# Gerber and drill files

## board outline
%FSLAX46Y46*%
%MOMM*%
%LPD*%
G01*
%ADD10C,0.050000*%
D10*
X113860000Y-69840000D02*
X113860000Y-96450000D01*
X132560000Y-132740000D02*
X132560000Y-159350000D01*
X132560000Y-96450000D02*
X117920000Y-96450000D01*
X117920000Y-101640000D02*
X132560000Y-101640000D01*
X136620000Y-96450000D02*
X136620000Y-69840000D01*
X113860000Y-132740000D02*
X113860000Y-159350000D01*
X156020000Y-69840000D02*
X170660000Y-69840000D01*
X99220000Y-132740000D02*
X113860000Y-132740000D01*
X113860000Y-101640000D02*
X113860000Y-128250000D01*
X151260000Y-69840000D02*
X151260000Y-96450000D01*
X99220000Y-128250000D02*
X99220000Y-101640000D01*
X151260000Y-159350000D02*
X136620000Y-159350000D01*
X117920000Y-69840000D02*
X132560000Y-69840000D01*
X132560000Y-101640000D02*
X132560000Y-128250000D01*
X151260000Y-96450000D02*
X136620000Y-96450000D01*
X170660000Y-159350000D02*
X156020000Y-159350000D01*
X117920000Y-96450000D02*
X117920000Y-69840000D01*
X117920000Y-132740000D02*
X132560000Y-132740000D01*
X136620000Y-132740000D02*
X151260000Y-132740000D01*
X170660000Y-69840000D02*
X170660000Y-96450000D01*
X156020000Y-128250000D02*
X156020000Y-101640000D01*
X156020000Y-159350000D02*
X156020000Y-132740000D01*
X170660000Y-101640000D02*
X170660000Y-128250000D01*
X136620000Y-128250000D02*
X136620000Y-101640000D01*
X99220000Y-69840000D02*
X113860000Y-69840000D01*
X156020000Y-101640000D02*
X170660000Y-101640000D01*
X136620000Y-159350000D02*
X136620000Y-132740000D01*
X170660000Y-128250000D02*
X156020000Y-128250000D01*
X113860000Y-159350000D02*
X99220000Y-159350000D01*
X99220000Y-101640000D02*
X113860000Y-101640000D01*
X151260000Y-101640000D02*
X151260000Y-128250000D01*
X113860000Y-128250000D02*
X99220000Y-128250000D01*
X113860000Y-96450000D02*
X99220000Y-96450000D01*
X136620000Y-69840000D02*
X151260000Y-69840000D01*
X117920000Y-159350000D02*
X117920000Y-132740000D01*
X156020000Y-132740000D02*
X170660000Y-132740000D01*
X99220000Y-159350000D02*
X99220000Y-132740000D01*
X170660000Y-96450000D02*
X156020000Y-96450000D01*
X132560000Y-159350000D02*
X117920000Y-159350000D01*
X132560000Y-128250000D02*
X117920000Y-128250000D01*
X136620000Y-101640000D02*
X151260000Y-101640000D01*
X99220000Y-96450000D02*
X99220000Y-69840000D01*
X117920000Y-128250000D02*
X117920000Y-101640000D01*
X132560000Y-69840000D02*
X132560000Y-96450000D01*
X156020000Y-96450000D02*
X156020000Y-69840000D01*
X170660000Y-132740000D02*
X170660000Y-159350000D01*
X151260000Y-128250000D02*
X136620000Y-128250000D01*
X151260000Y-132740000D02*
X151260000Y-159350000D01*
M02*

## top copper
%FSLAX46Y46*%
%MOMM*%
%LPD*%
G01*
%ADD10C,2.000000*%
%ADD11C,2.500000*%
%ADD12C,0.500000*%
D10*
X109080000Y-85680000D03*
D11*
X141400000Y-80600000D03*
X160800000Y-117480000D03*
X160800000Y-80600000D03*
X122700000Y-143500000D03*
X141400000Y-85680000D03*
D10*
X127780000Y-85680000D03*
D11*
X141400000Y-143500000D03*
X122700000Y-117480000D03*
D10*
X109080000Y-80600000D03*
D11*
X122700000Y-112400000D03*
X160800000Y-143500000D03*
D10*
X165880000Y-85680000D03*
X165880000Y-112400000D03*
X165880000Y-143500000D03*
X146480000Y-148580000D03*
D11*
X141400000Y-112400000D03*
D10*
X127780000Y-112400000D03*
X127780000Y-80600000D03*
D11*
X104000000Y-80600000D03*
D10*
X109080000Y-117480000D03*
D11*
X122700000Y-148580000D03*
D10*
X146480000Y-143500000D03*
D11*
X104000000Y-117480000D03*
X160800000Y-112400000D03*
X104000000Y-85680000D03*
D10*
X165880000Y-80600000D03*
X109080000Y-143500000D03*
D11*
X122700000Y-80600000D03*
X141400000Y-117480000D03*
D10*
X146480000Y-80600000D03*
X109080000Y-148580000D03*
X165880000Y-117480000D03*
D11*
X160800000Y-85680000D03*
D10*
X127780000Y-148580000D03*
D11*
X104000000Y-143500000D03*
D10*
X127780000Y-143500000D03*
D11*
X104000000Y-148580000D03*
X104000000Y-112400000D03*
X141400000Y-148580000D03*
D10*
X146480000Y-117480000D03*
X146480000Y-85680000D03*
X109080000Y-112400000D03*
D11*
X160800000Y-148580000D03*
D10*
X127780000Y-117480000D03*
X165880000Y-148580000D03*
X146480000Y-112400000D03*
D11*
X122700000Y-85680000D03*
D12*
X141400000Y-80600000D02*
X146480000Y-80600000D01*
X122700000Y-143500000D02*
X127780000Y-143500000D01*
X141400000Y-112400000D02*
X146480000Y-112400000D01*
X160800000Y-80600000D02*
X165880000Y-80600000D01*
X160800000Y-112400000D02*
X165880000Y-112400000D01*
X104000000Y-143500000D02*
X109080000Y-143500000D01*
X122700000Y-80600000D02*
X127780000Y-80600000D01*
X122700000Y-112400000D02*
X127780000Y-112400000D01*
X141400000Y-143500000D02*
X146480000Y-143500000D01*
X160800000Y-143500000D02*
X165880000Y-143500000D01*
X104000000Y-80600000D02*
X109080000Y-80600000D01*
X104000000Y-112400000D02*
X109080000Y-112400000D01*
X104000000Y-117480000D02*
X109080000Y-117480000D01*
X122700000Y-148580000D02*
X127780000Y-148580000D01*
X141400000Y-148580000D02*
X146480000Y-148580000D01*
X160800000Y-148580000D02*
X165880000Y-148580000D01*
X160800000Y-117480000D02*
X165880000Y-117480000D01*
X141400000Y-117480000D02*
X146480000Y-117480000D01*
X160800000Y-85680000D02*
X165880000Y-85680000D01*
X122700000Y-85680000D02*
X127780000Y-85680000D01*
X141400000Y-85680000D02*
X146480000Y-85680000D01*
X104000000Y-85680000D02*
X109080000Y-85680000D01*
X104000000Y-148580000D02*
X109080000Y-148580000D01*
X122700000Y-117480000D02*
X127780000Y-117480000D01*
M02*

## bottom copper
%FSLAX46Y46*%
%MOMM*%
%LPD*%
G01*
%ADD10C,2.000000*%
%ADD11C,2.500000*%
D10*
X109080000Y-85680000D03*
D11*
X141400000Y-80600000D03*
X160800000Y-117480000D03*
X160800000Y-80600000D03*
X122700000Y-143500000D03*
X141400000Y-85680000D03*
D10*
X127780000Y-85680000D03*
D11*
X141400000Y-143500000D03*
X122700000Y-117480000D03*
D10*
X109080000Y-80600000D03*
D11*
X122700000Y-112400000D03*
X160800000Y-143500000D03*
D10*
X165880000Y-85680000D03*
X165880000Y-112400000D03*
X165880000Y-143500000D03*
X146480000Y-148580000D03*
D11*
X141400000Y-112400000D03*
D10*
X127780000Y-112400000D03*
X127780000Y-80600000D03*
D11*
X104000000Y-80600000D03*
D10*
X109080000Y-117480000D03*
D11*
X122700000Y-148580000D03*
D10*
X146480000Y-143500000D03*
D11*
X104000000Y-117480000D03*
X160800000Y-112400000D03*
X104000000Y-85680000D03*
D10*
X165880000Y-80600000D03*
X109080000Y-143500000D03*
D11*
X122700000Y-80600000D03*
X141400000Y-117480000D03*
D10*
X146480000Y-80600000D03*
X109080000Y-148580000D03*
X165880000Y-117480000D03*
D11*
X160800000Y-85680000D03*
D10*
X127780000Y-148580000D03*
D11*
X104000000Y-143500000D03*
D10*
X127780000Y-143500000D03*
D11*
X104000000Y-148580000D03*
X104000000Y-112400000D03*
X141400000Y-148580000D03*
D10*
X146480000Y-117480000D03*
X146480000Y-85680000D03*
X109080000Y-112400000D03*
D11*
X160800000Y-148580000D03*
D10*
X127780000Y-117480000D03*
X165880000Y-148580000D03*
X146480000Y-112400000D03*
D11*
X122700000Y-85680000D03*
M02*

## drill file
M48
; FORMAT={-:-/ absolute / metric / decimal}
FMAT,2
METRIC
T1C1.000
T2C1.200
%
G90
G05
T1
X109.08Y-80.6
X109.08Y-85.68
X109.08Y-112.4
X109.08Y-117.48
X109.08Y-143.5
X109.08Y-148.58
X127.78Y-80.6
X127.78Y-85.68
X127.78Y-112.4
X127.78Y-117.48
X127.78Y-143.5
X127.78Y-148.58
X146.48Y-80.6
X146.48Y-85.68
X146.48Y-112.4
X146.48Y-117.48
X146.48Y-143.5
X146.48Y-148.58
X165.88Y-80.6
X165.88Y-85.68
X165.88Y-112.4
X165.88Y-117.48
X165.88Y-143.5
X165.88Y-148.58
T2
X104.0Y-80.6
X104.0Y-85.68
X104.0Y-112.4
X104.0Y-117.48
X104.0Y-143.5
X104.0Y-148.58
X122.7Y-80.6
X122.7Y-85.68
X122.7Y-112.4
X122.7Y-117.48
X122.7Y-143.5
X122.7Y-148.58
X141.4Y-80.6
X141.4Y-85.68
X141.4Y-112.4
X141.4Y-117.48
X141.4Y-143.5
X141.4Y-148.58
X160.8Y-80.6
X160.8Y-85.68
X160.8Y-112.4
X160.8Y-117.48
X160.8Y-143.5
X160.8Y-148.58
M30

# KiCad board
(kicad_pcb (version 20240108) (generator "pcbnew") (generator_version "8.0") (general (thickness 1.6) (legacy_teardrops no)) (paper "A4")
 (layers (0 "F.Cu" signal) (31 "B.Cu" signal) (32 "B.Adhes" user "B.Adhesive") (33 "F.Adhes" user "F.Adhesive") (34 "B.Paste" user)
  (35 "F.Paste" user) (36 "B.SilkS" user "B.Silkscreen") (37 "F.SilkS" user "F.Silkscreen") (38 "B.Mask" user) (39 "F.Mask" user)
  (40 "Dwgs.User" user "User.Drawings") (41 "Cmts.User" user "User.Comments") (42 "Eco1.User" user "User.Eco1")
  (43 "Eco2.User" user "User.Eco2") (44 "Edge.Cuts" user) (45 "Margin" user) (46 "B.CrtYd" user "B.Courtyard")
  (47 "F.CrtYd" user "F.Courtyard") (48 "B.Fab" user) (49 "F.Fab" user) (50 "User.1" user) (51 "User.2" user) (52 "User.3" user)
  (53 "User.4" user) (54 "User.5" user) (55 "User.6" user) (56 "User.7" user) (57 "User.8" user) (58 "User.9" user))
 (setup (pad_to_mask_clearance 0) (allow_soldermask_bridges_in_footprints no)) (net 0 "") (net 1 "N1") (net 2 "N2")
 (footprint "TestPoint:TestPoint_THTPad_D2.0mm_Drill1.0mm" (layer "F.Cu") (at 109.08 85.68)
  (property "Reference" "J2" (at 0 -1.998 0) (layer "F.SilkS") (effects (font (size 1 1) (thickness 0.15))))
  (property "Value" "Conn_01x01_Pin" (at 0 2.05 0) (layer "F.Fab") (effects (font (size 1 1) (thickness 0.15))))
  (pad "1" thru_hole circle (at 0 0) (size 2 2) (drill 1) (layers "*.Cu" "*.Mask") (remove_unused_layers no) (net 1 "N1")))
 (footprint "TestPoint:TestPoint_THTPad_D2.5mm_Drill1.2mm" (layer "F.Cu") (at 141.4 80.6)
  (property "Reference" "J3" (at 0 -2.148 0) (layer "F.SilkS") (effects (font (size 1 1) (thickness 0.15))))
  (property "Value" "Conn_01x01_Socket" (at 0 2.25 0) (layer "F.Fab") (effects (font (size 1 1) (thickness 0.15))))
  (pad "1" thru_hole circle (at 0 0) (size 2.5 2.5) (drill 1.2) (layers "*.Cu" "*.Mask") (remove_unused_layers no) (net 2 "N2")))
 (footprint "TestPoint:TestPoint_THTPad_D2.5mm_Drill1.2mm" (layer "F.Cu") (at 160.8 117.48)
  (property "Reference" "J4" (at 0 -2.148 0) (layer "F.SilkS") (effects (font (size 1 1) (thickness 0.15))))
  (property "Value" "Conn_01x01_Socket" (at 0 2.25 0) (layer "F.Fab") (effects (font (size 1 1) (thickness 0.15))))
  (pad "1" thru_hole circle (at 0 0) (size 2.5 2.5) (drill 1.2) (layers "*.Cu" "*.Mask") (remove_unused_layers no) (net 1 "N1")))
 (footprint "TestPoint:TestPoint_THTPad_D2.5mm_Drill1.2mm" (layer "F.Cu") (at 160.8 80.6)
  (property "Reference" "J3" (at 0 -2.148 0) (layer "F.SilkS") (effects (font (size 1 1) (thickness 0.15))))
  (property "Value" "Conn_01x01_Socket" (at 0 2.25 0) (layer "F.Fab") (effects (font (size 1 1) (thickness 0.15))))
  (pad "1" thru_hole circle (at 0 0) (size 2.5 2.5) (drill 1.2) (layers "*.Cu" "*.Mask") (remove_unused_layers no) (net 2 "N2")))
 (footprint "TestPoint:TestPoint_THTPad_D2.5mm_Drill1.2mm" (layer "F.Cu") (at 122.7 143.5)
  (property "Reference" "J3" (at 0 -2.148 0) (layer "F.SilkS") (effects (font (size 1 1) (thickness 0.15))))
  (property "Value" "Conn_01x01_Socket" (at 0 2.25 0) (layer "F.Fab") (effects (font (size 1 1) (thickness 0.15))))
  (pad "1" thru_hole circle (at 0 0) (size 2.5 2.5) (drill 1.2) (layers "*.Cu" "*.Mask") (remove_unused_layers no) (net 2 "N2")))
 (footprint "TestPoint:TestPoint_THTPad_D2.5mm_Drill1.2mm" (layer "F.Cu") (at 141.4 85.68)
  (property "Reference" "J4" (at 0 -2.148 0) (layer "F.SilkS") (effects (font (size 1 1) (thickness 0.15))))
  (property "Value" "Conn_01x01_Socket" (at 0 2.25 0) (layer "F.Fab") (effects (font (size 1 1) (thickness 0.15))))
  (pad "1" thru_hole circle (at 0 0) (size 2.5 2.5) (drill 1.2) (layers "*.Cu" "*.Mask") (remove_unused_layers no) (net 1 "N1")))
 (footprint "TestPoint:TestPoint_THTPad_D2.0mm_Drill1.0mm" (layer "F.Cu") (at 127.78 85.68)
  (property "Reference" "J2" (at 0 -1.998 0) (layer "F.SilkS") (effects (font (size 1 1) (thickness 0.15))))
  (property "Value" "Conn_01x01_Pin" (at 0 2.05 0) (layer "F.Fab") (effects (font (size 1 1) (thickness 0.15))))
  (pad "1" thru_hole circle (at 0 0) (size 2 2) (drill 1) (layers "*.Cu" "*.Mask") (remove_unused_layers no) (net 1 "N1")))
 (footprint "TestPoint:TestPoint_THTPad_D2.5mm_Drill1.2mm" (layer "F.Cu") (at 141.4 143.5)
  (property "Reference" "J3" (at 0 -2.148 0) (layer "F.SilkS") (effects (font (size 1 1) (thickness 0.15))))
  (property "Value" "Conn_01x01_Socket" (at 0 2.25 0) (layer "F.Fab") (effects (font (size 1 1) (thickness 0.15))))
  (pad "1" thru_hole circle (at 0 0) (size 2.5 2.5) (drill 1.2) (layers "*.Cu" "*.Mask") (remove_unused_layers no) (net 2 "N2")))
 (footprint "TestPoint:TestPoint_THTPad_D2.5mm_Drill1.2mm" (layer "F.Cu") (at 122.7 117.48)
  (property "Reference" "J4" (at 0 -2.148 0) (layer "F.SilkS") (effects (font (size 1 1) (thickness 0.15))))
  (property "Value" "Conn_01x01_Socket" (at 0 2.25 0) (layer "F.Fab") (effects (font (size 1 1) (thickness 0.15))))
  (pad "1" thru_hole circle (at 0 0) (size 2.5 2.5) (drill 1.2) (layers "*.Cu" "*.Mask") (remove_unused_layers no) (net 1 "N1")))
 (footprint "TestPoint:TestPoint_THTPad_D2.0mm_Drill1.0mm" (layer "F.Cu") (at 109.08 80.6)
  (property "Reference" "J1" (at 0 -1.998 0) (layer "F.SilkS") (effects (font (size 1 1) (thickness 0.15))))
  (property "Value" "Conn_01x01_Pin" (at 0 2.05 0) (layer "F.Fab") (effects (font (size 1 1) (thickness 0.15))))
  (pad "1" thru_hole circle (at 0 0) (size 2 2) (drill 1) (layers "*.Cu" "*.Mask") (remove_unused_layers no) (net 2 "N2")))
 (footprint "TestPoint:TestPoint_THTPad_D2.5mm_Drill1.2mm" (layer "F.Cu") (at 122.7 112.4)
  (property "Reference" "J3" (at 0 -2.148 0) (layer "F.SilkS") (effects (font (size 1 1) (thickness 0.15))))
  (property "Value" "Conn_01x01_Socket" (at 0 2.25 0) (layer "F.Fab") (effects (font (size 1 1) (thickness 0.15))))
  (pad "1" thru_hole circle (at 0 0) (size 2.5 2.5) (drill 1.2) (layers "*.Cu" "*.Mask") (remove_unused_layers no) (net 2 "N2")))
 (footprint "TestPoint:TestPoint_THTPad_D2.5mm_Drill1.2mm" (layer "F.Cu") (at 160.8 143.5)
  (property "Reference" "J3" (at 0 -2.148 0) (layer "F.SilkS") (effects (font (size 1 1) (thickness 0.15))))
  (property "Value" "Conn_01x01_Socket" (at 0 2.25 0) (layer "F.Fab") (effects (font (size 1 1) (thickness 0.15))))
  (pad "1" thru_hole circle (at 0 0) (size 2.5 2.5) (drill 1.2) (layers "*.Cu" "*.Mask") (remove_unused_layers no) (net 2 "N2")))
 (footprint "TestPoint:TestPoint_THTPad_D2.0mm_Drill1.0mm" (layer "F.Cu") (at 165.88 85.68)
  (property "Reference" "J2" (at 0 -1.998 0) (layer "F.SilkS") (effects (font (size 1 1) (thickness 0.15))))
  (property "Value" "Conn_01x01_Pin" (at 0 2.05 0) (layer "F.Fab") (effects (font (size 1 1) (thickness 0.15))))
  (pad "1" thru_hole circle (at 0 0) (size 2 2) (drill 1) (layers "*.Cu" "*.Mask") (remove_unused_layers no) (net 1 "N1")))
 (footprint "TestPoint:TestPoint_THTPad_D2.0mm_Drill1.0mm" (layer "F.Cu") (at 165.88 112.4)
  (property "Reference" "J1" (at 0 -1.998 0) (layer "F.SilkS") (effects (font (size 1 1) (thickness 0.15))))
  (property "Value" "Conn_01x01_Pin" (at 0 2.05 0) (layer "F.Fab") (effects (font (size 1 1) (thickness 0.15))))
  (pad "1" thru_hole circle (at 0 0) (size 2 2) (drill 1) (layers "*.Cu" "*.Mask") (remove_unused_layers no) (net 2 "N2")))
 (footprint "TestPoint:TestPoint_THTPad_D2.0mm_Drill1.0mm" (layer "F.Cu") (at 165.88 143.5)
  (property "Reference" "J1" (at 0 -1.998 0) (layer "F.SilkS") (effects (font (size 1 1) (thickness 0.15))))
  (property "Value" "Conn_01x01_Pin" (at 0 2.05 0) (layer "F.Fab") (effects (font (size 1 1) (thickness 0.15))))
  (pad "1" thru_hole circle (at 0 0) (size 2 2) (drill 1) (layers "*.Cu" "*.Mask") (remove_unused_layers no) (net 2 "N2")))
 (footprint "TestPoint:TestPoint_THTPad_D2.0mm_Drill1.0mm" (layer "F.Cu") (at 146.48 148.58)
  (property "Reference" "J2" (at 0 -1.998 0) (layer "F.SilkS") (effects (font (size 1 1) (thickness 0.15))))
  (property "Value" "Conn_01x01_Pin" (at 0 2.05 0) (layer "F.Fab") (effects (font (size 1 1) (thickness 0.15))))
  (pad "1" thru_hole circle (at 0 0) (size 2 2) (drill 1) (layers "*.Cu" "*.Mask") (remove_unused_layers no) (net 1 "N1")))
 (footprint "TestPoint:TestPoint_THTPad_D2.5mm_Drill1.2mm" (layer "F.Cu") (at 141.4 112.4)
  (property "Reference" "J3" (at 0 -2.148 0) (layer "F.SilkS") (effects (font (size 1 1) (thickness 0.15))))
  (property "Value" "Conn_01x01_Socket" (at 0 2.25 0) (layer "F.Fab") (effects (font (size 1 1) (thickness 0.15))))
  (pad "1" thru_hole circle (at 0 0) (size 2.5 2.5) (drill 1.2) (layers "*.Cu" "*.Mask") (remove_unused_layers no) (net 2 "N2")))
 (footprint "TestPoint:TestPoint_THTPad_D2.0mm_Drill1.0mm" (layer "F.Cu") (at 127.78 112.4)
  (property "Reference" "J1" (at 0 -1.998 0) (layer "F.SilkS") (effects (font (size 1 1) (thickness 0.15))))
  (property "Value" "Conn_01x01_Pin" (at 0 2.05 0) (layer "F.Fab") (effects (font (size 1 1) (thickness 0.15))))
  (pad "1" thru_hole circle (at 0 0) (size 2 2) (drill 1) (layers "*.Cu" "*.Mask") (remove_unused_layers no) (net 2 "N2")))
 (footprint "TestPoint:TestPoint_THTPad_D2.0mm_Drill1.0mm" (layer "F.Cu") (at 127.78 80.6)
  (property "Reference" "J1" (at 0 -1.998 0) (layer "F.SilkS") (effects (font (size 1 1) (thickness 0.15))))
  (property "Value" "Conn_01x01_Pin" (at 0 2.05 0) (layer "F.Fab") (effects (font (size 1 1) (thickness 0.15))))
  (pad "1" thru_hole circle (at 0 0) (size 2 2) (drill 1) (layers "*.Cu" "*.Mask") (remove_unused_layers no) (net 2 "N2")))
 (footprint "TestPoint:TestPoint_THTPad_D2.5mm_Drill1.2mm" (layer "F.Cu") (at 104 80.6)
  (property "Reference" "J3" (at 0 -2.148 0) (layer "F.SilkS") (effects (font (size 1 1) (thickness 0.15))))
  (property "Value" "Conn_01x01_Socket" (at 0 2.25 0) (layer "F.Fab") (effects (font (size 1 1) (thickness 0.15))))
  (pad "1" thru_hole circle (at 0 0) (size 2.5 2.5) (drill 1.2) (layers "*.Cu" "*.Mask") (remove_unused_layers no) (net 2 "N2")))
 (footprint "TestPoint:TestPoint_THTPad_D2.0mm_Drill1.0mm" (layer "F.Cu") (at 109.08 117.48)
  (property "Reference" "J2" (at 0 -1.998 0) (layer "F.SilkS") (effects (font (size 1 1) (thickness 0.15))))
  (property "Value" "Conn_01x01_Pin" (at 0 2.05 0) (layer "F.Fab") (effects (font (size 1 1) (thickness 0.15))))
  (pad "1" thru_hole circle (at 0 0) (size 2 2) (drill 1) (layers "*.Cu" "*.Mask") (remove_unused_layers no) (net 1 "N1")))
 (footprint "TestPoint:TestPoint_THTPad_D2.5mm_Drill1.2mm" (layer "F.Cu") (at 122.7 148.58)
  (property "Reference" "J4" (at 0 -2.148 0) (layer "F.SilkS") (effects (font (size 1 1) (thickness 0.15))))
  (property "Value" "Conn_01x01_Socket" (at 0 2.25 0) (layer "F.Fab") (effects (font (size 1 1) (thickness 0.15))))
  (pad "1" thru_hole circle (at 0 0) (size 2.5 2.5) (drill 1.2) (layers "*.Cu" "*.Mask") (remove_unused_layers no) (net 1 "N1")))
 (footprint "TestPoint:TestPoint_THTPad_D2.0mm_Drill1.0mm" (layer "F.Cu") (at 146.48 143.5)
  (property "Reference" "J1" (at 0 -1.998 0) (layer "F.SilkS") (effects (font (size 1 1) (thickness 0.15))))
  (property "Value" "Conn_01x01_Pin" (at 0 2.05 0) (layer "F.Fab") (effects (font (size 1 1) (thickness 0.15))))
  (pad "1" thru_hole circle (at 0 0) (size 2 2) (drill 1) (layers "*.Cu" "*.Mask") (remove_unused_layers no) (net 2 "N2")))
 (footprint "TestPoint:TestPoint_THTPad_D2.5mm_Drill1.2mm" (layer "F.Cu") (at 104 117.48)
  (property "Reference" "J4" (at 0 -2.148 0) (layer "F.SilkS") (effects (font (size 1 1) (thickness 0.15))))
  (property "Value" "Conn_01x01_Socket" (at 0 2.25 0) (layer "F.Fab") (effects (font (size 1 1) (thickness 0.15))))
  (pad "1" thru_hole circle (at 0 0) (size 2.5 2.5) (drill 1.2) (layers "*.Cu" "*.Mask") (remove_unused_layers no) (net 1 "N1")))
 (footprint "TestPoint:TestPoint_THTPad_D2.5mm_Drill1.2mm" (layer "F.Cu") (at 160.8 112.4)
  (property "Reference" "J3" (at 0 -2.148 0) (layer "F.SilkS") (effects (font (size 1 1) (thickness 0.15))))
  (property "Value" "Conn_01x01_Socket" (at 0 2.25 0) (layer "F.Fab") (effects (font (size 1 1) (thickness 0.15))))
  (pad "1" thru_hole circle (at 0 0) (size 2.5 2.5) (drill 1.2) (layers "*.Cu" "*.Mask") (remove_unused_layers no) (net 2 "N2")))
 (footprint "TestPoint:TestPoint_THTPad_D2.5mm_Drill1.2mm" (layer "F.Cu") (at 104 85.68)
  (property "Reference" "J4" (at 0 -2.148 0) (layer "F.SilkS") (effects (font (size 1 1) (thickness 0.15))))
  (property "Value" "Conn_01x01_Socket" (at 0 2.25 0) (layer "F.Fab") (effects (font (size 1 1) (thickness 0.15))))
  (pad "1" thru_hole circle (at 0 0) (size 2.5 2.5) (drill 1.2) (layers "*.Cu" "*.Mask") (remove_unused_layers no) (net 1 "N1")))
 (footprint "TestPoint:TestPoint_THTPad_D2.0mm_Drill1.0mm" (layer "F.Cu") (at 165.88 80.6)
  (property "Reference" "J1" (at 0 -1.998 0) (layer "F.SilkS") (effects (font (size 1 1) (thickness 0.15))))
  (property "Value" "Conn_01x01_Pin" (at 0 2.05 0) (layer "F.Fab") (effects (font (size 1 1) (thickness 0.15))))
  (pad "1" thru_hole circle (at 0 0) (size 2 2) (drill 1) (layers "*.Cu" "*.Mask") (remove_unused_layers no) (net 2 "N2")))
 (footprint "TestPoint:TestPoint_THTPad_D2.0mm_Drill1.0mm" (layer "F.Cu") (at 109.08 143.5)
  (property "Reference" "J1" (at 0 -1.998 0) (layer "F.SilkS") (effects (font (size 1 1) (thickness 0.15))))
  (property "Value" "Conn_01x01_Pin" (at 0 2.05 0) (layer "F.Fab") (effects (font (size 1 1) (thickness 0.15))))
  (pad "1" thru_hole circle (at 0 0) (size 2 2) (drill 1) (layers "*.Cu" "*.Mask") (remove_unused_layers no) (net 2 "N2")))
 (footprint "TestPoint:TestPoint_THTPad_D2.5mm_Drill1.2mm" (layer "F.Cu") (at 122.7 80.6)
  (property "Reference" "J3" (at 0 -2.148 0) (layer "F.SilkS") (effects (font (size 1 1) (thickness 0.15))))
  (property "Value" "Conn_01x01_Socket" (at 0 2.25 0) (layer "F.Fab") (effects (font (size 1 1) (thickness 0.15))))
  (pad "1" thru_hole circle (at 0 0) (size 2.5 2.5) (drill 1.2) (layers "*.Cu" "*.Mask") (remove_unused_layers no) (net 2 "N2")))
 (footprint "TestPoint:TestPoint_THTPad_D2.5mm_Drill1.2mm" (layer "F.Cu") (at 141.4 117.48)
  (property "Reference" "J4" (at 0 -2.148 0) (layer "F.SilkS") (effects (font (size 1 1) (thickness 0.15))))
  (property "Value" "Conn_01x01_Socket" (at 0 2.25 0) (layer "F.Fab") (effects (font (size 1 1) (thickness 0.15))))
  (pad "1" thru_hole circle (at 0 0) (size 2.5 2.5) (drill 1.2) (layers "*.Cu" "*.Mask") (remove_unused_layers no) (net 1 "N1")))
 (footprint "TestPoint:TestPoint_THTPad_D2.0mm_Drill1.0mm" (layer "F.Cu") (at 146.48 80.6)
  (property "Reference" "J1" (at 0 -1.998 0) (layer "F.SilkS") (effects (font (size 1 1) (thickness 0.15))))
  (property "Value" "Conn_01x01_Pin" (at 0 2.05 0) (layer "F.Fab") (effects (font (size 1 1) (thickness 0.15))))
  (pad "1" thru_hole circle (at 0 0) (size 2 2) (drill 1) (layers "*.Cu" "*.Mask") (remove_unused_layers no) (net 2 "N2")))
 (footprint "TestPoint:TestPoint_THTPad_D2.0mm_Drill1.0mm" (layer "F.Cu") (at 109.08 148.58)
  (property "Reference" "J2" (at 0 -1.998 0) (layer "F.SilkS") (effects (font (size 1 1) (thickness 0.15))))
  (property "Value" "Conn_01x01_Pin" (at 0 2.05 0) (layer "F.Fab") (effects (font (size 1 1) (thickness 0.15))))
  (pad "1" thru_hole circle (at 0 0) (size 2 2) (drill 1) (layers "*.Cu" "*.Mask") (remove_unused_layers no) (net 1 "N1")))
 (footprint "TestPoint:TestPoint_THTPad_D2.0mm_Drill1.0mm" (layer "F.Cu") (at 165.88 117.48)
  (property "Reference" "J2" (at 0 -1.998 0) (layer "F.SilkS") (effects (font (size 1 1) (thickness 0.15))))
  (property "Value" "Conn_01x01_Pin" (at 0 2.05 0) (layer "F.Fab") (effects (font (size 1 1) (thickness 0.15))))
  (pad "1" thru_hole circle (at 0 0) (size 2 2) (drill 1) (layers "*.Cu" "*.Mask") (remove_unused_layers no) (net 1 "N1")))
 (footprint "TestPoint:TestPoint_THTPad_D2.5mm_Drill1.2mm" (layer "F.Cu") (at 160.8 85.68)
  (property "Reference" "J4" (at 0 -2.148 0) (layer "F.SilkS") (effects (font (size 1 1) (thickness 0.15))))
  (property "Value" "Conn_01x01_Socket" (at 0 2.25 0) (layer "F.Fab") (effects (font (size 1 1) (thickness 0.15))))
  (pad "1" thru_hole circle (at 0 0) (size 2.5 2.5) (drill 1.2) (layers "*.Cu" "*.Mask") (remove_unused_layers no) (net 1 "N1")))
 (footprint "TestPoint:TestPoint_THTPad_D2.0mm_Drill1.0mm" (layer "F.Cu") (at 127.78 148.58)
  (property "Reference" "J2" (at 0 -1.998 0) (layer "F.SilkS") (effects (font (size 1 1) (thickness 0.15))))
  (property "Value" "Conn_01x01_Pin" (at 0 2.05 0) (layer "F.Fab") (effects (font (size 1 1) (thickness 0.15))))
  (pad "1" thru_hole circle (at 0 0) (size 2 2) (drill 1) (layers "*.Cu" "*.Mask") (remove_unused_layers no) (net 1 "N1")))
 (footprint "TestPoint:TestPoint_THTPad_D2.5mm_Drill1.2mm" (layer "F.Cu") (at 104 143.5)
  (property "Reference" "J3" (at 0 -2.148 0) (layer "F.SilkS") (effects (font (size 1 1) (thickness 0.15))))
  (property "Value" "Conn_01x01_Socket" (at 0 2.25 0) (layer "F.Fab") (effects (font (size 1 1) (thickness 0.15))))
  (pad "1" thru_hole circle (at 0 0) (size 2.5 2.5) (drill 1.2) (layers "*.Cu" "*.Mask") (remove_unused_layers no) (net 2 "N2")))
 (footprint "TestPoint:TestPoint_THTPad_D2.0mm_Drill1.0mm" (layer "F.Cu") (at 127.78 143.5)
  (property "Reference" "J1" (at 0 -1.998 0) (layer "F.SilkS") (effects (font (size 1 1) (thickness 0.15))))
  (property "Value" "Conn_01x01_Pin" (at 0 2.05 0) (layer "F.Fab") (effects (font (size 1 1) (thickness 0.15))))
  (pad "1" thru_hole circle (at 0 0) (size 2 2) (drill 1) (layers "*.Cu" "*.Mask") (remove_unused_layers no) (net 2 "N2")))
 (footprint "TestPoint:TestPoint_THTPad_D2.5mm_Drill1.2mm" (layer "F.Cu") (at 104 148.58)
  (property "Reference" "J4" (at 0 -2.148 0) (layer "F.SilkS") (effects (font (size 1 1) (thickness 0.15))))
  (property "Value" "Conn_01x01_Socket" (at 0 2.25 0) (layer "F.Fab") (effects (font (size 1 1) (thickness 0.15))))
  (pad "1" thru_hole circle (at 0 0) (size 2.5 2.5) (drill 1.2) (layers "*.Cu" "*.Mask") (remove_unused_layers no) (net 1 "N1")))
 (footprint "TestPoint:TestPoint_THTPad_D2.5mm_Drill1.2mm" (layer "F.Cu") (at 104 112.4)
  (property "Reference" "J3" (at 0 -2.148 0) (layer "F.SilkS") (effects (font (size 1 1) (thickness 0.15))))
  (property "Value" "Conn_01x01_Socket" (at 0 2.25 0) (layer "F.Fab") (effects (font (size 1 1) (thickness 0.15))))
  (pad "1" thru_hole circle (at 0 0) (size 2.5 2.5) (drill 1.2) (layers "*.Cu" "*.Mask") (remove_unused_layers no) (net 2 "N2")))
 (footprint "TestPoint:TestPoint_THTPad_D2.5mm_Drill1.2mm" (layer "F.Cu") (at 141.4 148.58)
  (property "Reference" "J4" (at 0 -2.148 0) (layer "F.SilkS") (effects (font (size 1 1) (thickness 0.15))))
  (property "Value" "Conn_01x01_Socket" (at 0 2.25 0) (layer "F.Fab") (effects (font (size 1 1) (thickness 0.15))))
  (pad "1" thru_hole circle (at 0 0) (size 2.5 2.5) (drill 1.2) (layers "*.Cu" "*.Mask") (remove_unused_layers no) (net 1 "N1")))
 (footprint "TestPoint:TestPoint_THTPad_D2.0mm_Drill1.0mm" (layer "F.Cu") (at 146.48 117.48)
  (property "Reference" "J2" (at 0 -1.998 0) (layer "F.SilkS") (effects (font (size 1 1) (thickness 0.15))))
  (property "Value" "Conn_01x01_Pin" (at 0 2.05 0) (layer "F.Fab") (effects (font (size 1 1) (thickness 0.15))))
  (pad "1" thru_hole circle (at 0 0) (size 2 2) (drill 1) (layers "*.Cu" "*.Mask") (remove_unused_layers no) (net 1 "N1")))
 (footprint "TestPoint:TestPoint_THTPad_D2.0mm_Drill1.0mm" (layer "F.Cu") (at 146.48 85.68)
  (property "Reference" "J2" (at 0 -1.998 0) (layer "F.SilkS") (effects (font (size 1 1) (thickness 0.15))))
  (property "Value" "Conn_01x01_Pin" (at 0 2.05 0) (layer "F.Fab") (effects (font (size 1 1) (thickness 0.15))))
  (pad "1" thru_hole circle (at 0 0) (size 2 2) (drill 1) (layers "*.Cu" "*.Mask") (remove_unused_layers no) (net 1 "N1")))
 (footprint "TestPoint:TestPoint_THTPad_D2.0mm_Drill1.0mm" (layer "F.Cu") (at 109.08 112.4)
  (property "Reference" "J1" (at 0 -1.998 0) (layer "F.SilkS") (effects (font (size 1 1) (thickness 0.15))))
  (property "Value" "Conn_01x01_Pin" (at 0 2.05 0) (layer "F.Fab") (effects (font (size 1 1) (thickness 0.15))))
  (pad "1" thru_hole circle (at 0 0) (size 2 2) (drill 1) (layers "*.Cu" "*.Mask") (remove_unused_layers no) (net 2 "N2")))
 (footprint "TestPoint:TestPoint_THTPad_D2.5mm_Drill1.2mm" (layer "F.Cu") (at 160.8 148.58)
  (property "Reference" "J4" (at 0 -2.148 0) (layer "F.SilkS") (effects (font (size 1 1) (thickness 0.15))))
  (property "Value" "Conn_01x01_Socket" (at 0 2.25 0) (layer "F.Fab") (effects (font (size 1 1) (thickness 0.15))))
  (pad "1" thru_hole circle (at 0 0) (size 2.5 2.5) (drill 1.2) (layers "*.Cu" "*.Mask") (remove_unused_layers no) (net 1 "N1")))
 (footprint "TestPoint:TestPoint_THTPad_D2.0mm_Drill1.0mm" (layer "F.Cu") (at 127.78 117.48)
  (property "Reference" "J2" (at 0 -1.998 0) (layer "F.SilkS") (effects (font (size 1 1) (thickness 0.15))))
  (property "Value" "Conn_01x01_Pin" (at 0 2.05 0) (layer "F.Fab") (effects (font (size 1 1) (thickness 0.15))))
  (pad "1" thru_hole circle (at 0 0) (size 2 2) (drill 1) (layers "*.Cu" "*.Mask") (remove_unused_layers no) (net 1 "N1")))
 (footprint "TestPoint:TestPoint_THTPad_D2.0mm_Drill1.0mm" (layer "F.Cu") (at 165.88 148.58)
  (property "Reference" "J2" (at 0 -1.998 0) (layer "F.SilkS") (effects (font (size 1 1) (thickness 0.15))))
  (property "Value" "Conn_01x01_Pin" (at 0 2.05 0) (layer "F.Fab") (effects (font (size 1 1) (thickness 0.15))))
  (pad "1" thru_hole circle (at 0 0) (size 2 2) (drill 1) (layers "*.Cu" "*.Mask") (remove_unused_layers no) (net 1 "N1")))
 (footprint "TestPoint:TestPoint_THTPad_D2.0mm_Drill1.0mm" (layer "F.Cu") (at 146.48 112.4)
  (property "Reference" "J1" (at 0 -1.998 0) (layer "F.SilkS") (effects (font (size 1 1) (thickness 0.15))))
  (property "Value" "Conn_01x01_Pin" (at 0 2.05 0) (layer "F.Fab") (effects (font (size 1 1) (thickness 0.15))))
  (pad "1" thru_hole circle (at 0 0) (size 2 2) (drill 1) (layers "*.Cu" "*.Mask") (remove_unused_layers no) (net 2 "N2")))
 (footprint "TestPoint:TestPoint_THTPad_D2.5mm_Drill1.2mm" (layer "F.Cu") (at 122.7 85.68)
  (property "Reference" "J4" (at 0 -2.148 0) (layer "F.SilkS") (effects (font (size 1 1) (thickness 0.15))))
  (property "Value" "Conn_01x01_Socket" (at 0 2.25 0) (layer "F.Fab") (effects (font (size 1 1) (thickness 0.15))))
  (pad "1" thru_hole circle (at 0 0) (size 2.5 2.5) (drill 1.2) (layers "*.Cu" "*.Mask") (remove_unused_layers no) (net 1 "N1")))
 (gr_line (start 113.86 69.84) (end 113.86 96.45) (stroke (width 0.05) (type default)) (layer "Edge.Cuts"))
 (gr_line (start 132.56 132.74) (end 132.56 159.35) (stroke (width 0.05) (type default)) (layer "Edge.Cuts"))
 (gr_line (start 132.56 96.45) (end 117.92 96.45) (stroke (width 0.05) (type default)) (layer "Edge.Cuts"))
 (gr_line (start 117.92 101.64) (end 132.56 101.64) (stroke (width 0.05) (type default)) (layer "Edge.Cuts"))
 (gr_line (start 136.62 96.45) (end 136.62 69.84) (stroke (width 0.05) (type default)) (layer "Edge.Cuts"))
 (gr_line (start 113.86 132.74) (end 113.86 159.35) (stroke (width 0.05) (type default)) (layer "Edge.Cuts"))
 (gr_line (start 156.02 69.84) (end 170.66 69.84) (stroke (width 0.05) (type default)) (layer "Edge.Cuts"))
 (gr_line (start 99.22 132.74) (end 113.86 132.74) (stroke (width 0.05) (type default)) (layer "Edge.Cuts"))
 (gr_line (start 113.86 101.64) (end 113.86 128.25) (stroke (width 0.05) (type default)) (layer "Edge.Cuts"))
 (gr_line (start 151.26 69.84) (end 151.26 96.45) (stroke (width 0.05) (type default)) (layer "Edge.Cuts"))
 (gr_line (start 99.22 128.25) (end 99.22 101.64) (stroke (width 0.05) (type default)) (layer "Edge.Cuts"))
 (gr_line (start 151.26 159.35) (end 136.62 159.35) (stroke (width 0.05) (type default)) (layer "Edge.Cuts"))
 (gr_line (start 117.92 69.84) (end 132.56 69.84) (stroke (width 0.05) (type default)) (layer "Edge.Cuts"))
 (gr_line (start 132.56 101.64) (end 132.56 128.25) (stroke (width 0.05) (type default)) (layer "Edge.Cuts"))
 (gr_line (start 151.26 96.45) (end 136.62 96.45) (stroke (width 0.05) (type default)) (layer "Edge.Cuts"))
 (gr_line (start 170.66 159.35) (end 156.02 159.35) (stroke (width 0.05) (type default)) (layer "Edge.Cuts"))
 (gr_line (start 117.92 96.45) (end 117.92 69.84) (stroke (width 0.05) (type default)) (layer "Edge.Cuts"))
 (gr_line (start 117.92 132.74) (end 132.56 132.74) (stroke (width 0.05) (type default)) (layer "Edge.Cuts"))
 (gr_line (start 136.62 132.74) (end 151.26 132.74) (stroke (width 0.05) (type default)) (layer "Edge.Cuts"))
 (gr_line (start 170.66 69.84) (end 170.66 96.45) (stroke (width 0.05) (type default)) (layer "Edge.Cuts"))
 (gr_line (start 156.02 128.25) (end 156.02 101.64) (stroke (width 0.05) (type default)) (layer "Edge.Cuts"))
 (gr_line (start 156.02 159.35) (end 156.02 132.74) (stroke (width 0.05) (type default)) (layer "Edge.Cuts"))
 (gr_line (start 170.66 101.64) (end 170.66 128.25) (stroke (width 0.05) (type default)) (layer "Edge.Cuts"))
 (gr_line (start 136.62 128.25) (end 136.62 101.64) (stroke (width 0.05) (type default)) (layer "Edge.Cuts"))
 (gr_line (start 99.22 69.84) (end 113.86 69.84) (stroke (width 0.05) (type default)) (layer "Edge.Cuts"))
 (gr_line (start 156.02 101.64) (end 170.66 101.64) (stroke (width 0.05) (type default)) (layer "Edge.Cuts"))
 (gr_line (start 136.62 159.35) (end 136.62 132.74) (stroke (width 0.05) (type default)) (layer "Edge.Cuts"))
 (gr_line (start 170.66 128.25) (end 156.02 128.25) (stroke (width 0.05) (type default)) (layer "Edge.Cuts"))
 (gr_line (start 113.86 159.35) (end 99.22 159.35) (stroke (width 0.05) (type default)) (layer "Edge.Cuts"))
 (gr_line (start 99.22 101.64) (end 113.86 101.64) (stroke (width 0.05) (type default)) (layer "Edge.Cuts"))
 (gr_line (start 151.26 101.64) (end 151.26 128.25) (stroke (width 0.05) (type default)) (layer "Edge.Cuts"))
 (gr_line (start 113.86 128.25) (end 99.22 128.25) (stroke (width 0.05) (type default)) (layer "Edge.Cuts"))
 (gr_line (start 113.86 96.45) (end 99.22 96.45) (stroke (width 0.05) (type default)) (layer "Edge.Cuts"))
 (gr_line (start 136.62 69.84) (end 151.26 69.84) (stroke (width 0.05) (type default)) (layer "Edge.Cuts"))
 (gr_line (start 117.92 159.35) (end 117.92 132.74) (stroke (width 0.05) (type default)) (layer "Edge.Cuts"))
 (gr_line (start 156.02 132.74) (end 170.66 132.74) (stroke (width 0.05) (type default)) (layer "Edge.Cuts"))
 (gr_line (start 99.22 159.35) (end 99.22 132.74) (stroke (width 0.05) (type default)) (layer "Edge.Cuts"))
 (gr_line (start 170.66 96.45) (end 156.02 96.45) (stroke (width 0.05) (type default)) (layer "Edge.Cuts"))
 (gr_line (start 132.56 159.35) (end 117.92 159.35) (stroke (width 0.05) (type default)) (layer "Edge.Cuts"))
 (gr_line (start 132.56 128.25) (end 117.92 128.25) (stroke (width 0.05) (type default)) (layer "Edge.Cuts"))
 (gr_line (start 136.62 101.64) (end 151.26 101.64) (stroke (width 0.05) (type default)) (layer "Edge.Cuts"))
 (gr_line (start 99.22 96.45) (end 99.22 69.84) (stroke (width 0.05) (type default)) (layer "Edge.Cuts"))
 (gr_line (start 117.92 128.25) (end 117.92 101.64) (stroke (width 0.05) (type default)) (layer "Edge.Cuts"))
 (gr_line (start 132.56 69.84) (end 132.56 96.45) (stroke (width 0.05) (type default)) (layer "Edge.Cuts"))
 (gr_line (start 156.02 96.45) (end 156.02 69.84) (stroke (width 0.05) (type default)) (layer "Edge.Cuts"))
 (gr_line (start 170.66 132.74) (end 170.66 159.35) (stroke (width 0.05) (type default)) (layer "Edge.Cuts"))
 (gr_line (start 151.26 128.25) (end 136.62 128.25) (stroke (width 0.05) (type default)) (layer "Edge.Cuts"))
 (gr_line (start 151.26 132.74) (end 151.26 159.35) (stroke (width 0.05) (type default)) (layer "Edge.Cuts"))
 (segment (start 141.4 80.6) (end 146.48 80.6) (width 0.5) (layer "F.Cu") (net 2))
 (segment (start 122.7 143.5) (end 127.78 143.5) (width 0.5) (layer "F.Cu") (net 2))
 (segment (start 141.4 112.4) (end 146.48 112.4) (width 0.5) (layer "F.Cu") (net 2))
 (segment (start 160.8 80.6) (end 165.88 80.6) (width 0.5) (layer "F.Cu") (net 2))
 (segment (start 160.8 112.4) (end 165.88 112.4) (width 0.5) (layer "F.Cu") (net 2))
 (segment (start 104 143.5) (end 109.08 143.5) (width 0.5) (layer "F.Cu") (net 2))
 (segment (start 122.7 80.6) (end 127.78 80.6) (width 0.5) (layer "F.Cu") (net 2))
 (segment (start 122.7 112.4) (end 127.78 112.4) (width 0.5) (layer "F.Cu") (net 2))
 (segment (start 141.4 143.5) (end 146.48 143.5) (width 0.5) (layer "F.Cu") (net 2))
 (segment (start 160.8 143.5) (end 165.88 143.5) (width 0.5) (layer "F.Cu") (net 2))
 (segment (start 104 80.6) (end 109.08 80.6) (width 0.5) (layer "F.Cu") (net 2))
 (segment (start 104 112.4) (end 109.08 112.4) (width 0.5) (layer "F.Cu") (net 2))
 (segment (start 104 117.48) (end 109.08 117.48) (width 0.5) (layer "F.Cu") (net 1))
 (segment (start 122.7 148.58) (end 127.78 148.58) (width 0.5) (layer "F.Cu") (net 1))
 (segment (start 141.4 148.58) (end 146.48 148.58) (width 0.5) (layer "F.Cu") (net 1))
 (segment (start 160.8 148.58) (end 165.88 148.58) (width 0.5) (layer "F.Cu") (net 1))
 (segment (start 160.8 117.48) (end 165.88 117.48) (width 0.5) (layer "F.Cu") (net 1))
 (segment (start 141.4 117.48) (end 146.48 117.48) (width 0.5) (layer "F.Cu") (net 1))
 (segment (start 160.8 85.68) (end 165.88 85.68) (width 0.5) (layer "F.Cu") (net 1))
 (segment (start 122.7 85.68) (end 127.78 85.68) (width 0.5) (layer "F.Cu") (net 1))
 (segment (start 141.4 85.68) (end 146.48 85.68) (width 0.5) (layer "F.Cu") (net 1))
 (segment (start 104 85.68) (end 109.08 85.68) (width 0.5) (layer "F.Cu") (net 1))
 (segment (start 104 148.58) (end 109.08 148.58) (width 0.5) (layer "F.Cu") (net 1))
 (segment (start 122.7 117.48) (end 127.78 117.48) (width 0.5) (layer "F.Cu") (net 1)))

